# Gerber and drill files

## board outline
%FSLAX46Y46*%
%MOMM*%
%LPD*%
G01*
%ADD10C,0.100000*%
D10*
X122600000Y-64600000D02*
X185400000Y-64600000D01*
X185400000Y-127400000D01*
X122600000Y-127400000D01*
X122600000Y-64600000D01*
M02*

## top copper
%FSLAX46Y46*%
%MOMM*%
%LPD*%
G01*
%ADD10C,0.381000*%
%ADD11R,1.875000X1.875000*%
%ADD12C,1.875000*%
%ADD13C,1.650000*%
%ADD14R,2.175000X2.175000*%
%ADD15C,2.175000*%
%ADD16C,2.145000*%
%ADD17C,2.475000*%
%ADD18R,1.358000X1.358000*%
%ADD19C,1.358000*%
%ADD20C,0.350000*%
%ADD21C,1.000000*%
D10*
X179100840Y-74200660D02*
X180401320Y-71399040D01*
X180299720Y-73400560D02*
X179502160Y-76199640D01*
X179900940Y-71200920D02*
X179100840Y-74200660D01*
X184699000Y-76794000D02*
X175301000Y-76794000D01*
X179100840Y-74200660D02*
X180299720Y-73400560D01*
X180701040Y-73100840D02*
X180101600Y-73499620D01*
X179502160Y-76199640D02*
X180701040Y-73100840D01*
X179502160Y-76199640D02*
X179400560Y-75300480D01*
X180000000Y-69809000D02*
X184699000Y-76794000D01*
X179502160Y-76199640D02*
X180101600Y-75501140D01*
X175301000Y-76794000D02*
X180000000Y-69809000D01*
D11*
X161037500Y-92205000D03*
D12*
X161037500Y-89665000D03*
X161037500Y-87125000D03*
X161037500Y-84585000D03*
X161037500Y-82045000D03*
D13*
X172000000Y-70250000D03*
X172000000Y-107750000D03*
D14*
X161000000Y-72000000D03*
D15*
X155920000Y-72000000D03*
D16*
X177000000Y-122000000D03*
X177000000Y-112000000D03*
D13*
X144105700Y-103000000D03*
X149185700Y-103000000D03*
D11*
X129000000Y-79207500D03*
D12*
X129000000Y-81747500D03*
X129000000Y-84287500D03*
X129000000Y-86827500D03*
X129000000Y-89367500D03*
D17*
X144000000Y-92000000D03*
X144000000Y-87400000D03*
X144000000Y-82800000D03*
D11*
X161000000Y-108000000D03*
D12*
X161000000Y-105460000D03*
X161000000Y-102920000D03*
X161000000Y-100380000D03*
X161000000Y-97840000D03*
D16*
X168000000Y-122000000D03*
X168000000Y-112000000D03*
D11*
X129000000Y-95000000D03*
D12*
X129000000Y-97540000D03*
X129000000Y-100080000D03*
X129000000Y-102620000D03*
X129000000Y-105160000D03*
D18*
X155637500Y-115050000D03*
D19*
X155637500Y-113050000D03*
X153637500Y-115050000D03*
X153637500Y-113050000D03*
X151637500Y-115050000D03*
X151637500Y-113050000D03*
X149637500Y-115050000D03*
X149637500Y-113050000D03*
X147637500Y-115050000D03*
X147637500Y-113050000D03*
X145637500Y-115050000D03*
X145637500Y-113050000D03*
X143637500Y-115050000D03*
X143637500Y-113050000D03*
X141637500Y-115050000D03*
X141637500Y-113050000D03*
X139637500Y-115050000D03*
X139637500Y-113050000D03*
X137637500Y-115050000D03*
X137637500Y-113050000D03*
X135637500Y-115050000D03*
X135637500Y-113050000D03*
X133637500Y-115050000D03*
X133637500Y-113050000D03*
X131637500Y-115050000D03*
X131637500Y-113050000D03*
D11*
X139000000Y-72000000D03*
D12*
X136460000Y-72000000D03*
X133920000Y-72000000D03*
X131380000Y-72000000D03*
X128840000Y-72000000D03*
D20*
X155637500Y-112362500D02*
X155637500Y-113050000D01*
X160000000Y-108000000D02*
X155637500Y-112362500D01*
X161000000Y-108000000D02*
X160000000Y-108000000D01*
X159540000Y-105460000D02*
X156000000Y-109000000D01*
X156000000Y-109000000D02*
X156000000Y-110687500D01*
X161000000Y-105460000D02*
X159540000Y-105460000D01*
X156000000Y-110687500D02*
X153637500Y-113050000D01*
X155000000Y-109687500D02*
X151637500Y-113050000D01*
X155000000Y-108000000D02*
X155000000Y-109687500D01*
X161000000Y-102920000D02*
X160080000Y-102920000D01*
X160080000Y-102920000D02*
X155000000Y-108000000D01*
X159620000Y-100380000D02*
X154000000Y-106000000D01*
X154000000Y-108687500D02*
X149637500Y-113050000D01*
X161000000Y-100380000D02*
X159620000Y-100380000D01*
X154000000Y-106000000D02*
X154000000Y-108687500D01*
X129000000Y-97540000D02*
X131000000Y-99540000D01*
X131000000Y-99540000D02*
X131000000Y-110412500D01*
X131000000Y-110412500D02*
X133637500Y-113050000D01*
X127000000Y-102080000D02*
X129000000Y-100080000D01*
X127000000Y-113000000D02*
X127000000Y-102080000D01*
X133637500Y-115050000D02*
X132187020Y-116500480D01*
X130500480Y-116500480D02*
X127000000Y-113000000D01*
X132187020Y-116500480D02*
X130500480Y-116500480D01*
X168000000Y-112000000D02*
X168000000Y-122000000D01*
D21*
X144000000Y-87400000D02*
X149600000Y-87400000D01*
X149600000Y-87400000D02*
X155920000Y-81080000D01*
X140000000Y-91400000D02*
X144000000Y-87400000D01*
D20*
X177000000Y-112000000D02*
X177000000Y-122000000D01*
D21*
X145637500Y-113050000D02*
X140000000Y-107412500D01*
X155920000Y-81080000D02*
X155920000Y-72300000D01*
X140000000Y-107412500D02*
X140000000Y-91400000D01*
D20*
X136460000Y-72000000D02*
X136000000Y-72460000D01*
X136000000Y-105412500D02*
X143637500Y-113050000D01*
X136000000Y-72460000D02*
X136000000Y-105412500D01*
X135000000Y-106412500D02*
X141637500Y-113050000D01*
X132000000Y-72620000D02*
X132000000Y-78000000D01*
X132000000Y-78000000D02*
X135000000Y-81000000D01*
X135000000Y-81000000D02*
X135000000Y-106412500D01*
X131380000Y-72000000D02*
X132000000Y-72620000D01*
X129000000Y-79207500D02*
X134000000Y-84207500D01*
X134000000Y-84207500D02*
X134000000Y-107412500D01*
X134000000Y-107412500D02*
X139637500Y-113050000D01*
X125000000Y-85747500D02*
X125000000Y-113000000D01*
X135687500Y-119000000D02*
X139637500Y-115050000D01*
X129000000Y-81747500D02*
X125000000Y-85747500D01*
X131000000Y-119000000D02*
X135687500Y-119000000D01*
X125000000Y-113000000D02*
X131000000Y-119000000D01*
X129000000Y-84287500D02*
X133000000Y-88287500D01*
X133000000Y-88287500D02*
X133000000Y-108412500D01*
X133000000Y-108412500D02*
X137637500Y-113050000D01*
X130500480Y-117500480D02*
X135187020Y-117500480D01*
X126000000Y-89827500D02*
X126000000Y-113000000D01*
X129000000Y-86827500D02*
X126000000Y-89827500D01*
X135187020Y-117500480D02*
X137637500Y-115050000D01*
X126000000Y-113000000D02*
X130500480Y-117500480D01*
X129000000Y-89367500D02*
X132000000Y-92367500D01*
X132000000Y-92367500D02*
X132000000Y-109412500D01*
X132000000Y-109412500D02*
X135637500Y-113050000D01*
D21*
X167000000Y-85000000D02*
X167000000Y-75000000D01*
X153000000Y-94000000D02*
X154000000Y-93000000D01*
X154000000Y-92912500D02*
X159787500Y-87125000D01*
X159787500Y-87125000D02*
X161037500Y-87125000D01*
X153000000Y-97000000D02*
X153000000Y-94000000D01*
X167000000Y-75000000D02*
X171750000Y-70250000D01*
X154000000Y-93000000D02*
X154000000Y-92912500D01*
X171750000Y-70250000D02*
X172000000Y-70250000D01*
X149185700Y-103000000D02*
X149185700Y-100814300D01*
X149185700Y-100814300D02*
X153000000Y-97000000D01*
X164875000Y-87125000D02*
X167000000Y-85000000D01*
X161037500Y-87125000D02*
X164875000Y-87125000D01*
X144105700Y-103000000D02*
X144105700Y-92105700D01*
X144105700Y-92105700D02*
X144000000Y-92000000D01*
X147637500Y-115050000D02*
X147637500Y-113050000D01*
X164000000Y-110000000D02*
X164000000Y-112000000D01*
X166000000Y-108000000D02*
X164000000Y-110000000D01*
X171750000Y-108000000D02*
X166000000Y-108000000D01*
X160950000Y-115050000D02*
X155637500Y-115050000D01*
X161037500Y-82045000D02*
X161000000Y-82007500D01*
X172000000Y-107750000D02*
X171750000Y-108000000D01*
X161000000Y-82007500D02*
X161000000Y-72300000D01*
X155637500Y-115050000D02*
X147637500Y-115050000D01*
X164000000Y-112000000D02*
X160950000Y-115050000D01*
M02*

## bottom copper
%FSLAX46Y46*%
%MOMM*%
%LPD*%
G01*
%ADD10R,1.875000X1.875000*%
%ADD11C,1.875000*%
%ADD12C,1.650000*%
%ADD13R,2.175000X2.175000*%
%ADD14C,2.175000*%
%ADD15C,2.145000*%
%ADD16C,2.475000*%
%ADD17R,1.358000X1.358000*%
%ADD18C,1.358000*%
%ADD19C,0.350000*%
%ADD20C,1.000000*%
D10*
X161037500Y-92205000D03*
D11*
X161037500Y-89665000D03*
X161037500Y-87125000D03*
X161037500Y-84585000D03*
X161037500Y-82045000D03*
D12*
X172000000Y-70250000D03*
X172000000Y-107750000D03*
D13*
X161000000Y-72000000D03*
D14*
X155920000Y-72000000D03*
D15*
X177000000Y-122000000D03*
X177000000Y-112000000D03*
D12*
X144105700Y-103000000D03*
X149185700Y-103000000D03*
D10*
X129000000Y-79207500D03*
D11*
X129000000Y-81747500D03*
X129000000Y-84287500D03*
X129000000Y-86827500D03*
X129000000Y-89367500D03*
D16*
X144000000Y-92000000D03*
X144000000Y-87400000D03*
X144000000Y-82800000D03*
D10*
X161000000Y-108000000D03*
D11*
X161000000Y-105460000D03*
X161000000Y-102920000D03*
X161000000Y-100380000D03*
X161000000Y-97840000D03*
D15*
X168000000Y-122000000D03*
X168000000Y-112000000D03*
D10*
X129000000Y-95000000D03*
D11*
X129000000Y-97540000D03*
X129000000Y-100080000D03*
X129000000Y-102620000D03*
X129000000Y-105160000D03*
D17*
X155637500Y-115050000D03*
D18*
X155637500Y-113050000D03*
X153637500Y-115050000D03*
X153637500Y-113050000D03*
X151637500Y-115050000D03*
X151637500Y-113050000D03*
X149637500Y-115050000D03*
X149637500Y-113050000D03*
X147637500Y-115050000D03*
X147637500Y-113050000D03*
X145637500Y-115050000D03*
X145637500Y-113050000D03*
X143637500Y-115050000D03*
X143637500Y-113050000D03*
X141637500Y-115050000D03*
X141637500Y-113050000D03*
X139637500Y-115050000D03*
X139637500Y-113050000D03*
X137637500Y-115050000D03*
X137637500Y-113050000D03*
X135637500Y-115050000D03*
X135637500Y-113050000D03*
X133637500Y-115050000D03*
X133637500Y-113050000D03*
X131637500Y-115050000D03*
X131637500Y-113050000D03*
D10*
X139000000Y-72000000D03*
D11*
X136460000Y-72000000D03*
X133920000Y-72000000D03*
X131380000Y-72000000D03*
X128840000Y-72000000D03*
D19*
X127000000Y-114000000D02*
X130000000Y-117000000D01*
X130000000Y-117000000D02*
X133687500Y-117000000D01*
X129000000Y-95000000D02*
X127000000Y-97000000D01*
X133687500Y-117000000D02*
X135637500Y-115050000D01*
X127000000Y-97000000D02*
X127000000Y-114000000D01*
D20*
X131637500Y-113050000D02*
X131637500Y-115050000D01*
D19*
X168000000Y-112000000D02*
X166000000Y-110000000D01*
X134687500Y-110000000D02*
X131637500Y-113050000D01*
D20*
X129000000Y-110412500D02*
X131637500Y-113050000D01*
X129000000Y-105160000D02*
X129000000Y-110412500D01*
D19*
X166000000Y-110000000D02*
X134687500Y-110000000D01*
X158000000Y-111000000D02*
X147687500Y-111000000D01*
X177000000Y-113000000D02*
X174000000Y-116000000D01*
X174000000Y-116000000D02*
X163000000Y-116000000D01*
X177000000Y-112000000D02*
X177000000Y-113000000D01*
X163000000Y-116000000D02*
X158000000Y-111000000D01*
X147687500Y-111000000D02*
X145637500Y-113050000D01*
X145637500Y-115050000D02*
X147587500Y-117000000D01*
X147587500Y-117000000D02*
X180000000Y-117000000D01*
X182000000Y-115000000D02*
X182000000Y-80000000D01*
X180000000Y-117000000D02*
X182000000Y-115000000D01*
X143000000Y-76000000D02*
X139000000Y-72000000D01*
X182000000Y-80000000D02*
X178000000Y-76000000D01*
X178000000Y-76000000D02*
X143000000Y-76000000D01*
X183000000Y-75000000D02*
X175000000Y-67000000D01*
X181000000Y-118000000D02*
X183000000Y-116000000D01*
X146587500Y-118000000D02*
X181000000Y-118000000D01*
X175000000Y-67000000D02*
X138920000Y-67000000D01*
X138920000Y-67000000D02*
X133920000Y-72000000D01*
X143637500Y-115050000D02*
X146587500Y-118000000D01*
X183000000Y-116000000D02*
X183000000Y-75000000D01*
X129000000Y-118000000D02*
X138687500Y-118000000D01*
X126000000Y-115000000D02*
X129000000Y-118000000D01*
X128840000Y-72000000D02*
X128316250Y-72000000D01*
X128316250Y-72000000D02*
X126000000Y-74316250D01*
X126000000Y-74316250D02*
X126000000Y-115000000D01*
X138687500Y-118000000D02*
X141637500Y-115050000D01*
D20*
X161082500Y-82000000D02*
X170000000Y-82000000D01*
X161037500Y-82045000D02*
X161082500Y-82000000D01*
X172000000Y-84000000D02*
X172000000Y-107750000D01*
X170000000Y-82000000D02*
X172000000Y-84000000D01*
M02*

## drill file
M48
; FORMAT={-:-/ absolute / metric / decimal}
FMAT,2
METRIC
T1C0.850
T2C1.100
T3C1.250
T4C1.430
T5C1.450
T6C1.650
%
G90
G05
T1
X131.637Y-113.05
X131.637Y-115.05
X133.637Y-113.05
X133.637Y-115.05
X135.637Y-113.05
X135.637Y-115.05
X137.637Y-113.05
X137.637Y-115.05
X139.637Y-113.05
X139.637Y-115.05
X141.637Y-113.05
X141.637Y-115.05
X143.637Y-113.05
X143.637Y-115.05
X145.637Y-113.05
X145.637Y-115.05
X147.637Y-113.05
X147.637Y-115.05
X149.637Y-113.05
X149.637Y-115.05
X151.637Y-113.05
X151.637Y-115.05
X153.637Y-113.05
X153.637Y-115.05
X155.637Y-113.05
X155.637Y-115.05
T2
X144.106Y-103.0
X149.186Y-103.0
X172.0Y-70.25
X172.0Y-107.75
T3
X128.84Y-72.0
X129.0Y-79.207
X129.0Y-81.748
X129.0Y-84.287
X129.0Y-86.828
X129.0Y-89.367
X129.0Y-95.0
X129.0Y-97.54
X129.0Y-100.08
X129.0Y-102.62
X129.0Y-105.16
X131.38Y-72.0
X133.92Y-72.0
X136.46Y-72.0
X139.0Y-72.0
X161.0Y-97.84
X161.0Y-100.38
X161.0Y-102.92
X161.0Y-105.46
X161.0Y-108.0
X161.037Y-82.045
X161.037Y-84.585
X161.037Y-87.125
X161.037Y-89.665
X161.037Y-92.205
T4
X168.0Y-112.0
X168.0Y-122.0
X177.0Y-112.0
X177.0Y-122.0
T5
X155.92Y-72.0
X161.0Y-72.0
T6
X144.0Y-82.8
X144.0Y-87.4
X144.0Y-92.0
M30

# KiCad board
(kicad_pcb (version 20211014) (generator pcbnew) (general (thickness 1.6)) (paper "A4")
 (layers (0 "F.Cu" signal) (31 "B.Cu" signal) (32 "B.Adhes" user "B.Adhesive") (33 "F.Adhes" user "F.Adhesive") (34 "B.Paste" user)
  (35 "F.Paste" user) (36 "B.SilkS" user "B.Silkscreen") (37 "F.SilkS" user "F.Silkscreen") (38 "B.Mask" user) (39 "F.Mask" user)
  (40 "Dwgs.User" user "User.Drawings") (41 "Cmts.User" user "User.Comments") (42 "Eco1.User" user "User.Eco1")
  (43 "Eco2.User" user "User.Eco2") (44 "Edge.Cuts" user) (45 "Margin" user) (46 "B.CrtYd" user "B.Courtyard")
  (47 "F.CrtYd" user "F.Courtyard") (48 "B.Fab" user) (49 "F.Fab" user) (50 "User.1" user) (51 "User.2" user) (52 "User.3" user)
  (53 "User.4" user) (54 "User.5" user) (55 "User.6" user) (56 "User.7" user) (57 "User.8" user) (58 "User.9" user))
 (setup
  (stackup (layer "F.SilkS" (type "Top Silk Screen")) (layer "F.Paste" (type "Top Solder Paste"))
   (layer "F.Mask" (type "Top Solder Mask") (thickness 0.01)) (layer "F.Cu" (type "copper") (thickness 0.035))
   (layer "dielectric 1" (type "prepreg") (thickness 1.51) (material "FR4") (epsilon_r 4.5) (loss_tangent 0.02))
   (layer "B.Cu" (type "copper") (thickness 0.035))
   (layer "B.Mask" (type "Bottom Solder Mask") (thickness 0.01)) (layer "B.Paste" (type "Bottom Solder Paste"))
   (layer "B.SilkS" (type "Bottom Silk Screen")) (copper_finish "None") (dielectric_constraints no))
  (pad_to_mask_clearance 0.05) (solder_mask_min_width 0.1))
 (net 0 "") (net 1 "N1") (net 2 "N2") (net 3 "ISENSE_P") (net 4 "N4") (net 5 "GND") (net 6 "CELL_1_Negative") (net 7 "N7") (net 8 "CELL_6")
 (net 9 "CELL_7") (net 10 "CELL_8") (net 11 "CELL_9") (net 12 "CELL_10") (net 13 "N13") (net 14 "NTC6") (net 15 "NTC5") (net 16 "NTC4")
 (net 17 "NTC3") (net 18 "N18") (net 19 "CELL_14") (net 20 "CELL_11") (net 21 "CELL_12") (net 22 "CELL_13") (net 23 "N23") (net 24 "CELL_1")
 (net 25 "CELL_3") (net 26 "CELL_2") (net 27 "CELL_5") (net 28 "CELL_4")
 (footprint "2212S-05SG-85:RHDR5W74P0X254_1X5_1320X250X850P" (layer "F.Cu") (at 161.0375 92.205 90)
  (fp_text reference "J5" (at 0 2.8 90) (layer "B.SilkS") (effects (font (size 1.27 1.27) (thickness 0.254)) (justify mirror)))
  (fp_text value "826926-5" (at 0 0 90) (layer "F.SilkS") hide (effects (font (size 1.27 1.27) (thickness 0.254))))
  (pad "1" thru_hole rect locked (at 0 0 90) (size 1.875 1.875) (drill 1.25) (layers *.Cu *.Mask) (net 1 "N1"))
  (pad "2" thru_hole circle locked (at 2.54 0 90) (size 1.875 1.875) (drill 1.25) (layers *.Cu *.Mask) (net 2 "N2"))
  (pad "3" thru_hole circle locked (at 5.08 0 90) (size 1.875 1.875) (drill 1.25) (layers *.Cu *.Mask) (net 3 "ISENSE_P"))
  (pad "4" thru_hole circle locked (at 7.62 0 90) (size 1.875 1.875) (drill 1.25) (layers *.Cu *.Mask) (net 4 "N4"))
  (pad "5" thru_hole circle locked (at 10.16 0 90) (size 1.875 1.875) (drill 1.25) (layers *.Cu *.Mask) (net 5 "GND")))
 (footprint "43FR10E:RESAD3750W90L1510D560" (layer "F.Cu") (at 172 70.25 -90)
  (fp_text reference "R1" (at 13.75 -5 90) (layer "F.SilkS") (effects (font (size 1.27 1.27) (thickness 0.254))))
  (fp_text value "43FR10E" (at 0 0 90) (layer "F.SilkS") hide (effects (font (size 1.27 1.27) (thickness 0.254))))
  (pad "1" thru_hole circle locked (at 0 0 270) (size 1.65 1.65) (drill 1.1) (layers *.Cu *.Mask) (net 3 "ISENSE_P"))
  (pad "2" thru_hole circle locked (at 37.5 0 270) (size 1.65 1.65) (drill 1.1) (layers *.Cu *.Mask) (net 5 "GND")))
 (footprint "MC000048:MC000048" (layer "F.Cu") (at 161 72 180)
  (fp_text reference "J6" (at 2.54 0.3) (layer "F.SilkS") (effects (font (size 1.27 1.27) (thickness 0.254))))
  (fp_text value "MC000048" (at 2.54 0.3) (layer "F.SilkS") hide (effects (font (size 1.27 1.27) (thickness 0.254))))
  (pad "1" thru_hole rect locked (at 0 0 180) (size 2.175 2.175) (drill 1.45) (layers *.Cu *.Mask) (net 5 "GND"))
  (pad "2" thru_hole circle locked (at 5.08 0 180) (size 2.175 2.175) (drill 1.45) (layers *.Cu *.Mask) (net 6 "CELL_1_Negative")))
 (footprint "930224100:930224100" (layer "F.Cu") (at 177 122 90)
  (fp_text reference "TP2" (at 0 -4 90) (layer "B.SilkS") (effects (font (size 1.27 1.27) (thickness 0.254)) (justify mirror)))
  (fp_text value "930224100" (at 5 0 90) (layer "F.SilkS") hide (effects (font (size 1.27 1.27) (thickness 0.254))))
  (pad "1" thru_hole circle locked (at 0 0 90) (size 2.145 2.145) (drill 1.43) (layers *.Cu *.Mask) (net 6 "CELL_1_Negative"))
  (pad "2" thru_hole circle locked (at 10 0 90) (size 2.145 2.145) (drill 1.43) (layers *.Cu *.Mask) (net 6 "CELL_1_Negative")))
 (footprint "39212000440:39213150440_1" (layer "F.Cu") (at 146.6457 103)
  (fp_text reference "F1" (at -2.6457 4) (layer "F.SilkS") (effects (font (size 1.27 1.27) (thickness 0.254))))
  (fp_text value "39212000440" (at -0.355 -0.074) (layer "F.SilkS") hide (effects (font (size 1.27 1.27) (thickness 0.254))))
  (pad "1" thru_hole circle locked (at -2.54 0) (size 1.65 1.65) (drill 1.1) (layers *.Cu *.Mask) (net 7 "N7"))
  (pad "2" thru_hole circle locked (at 2.54 0) (size 1.65 1.65) (drill 1.1) (layers *.Cu *.Mask) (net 3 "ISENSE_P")))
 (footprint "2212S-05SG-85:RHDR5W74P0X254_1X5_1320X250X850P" (layer "F.Cu") (at 129 79.2075 -90)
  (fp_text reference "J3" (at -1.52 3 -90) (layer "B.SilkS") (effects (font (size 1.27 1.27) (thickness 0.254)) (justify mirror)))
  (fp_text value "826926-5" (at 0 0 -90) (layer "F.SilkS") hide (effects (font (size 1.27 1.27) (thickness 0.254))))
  (pad "1" thru_hole rect locked (at 0 0 270) (size 1.875 1.875) (drill 1.25) (layers *.Cu *.Mask) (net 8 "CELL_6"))
  (pad "2" thru_hole circle locked (at 2.54 0 270) (size 1.875 1.875) (drill 1.25) (layers *.Cu *.Mask) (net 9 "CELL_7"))
  (pad "3" thru_hole circle locked (at 5.08 0 270) (size 1.875 1.875) (drill 1.25) (layers *.Cu *.Mask) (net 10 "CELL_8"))
  (pad "4" thru_hole circle locked (at 7.62 0 270) (size 1.875 1.875) (drill 1.25) (layers *.Cu *.Mask) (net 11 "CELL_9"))
  (pad "5" thru_hole circle locked (at 10.16 0 270) (size 1.875 1.875) (drill 1.25) (layers *.Cu *.Mask) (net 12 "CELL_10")))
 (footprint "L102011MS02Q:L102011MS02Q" (layer "F.Cu") (at 144 92)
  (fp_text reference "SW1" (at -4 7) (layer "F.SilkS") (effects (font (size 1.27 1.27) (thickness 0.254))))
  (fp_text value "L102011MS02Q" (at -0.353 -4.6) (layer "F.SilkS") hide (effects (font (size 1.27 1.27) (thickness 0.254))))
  (pad "1" thru_hole circle locked (at 0 0) (size 2.475 2.475) (drill 1.65) (layers *.Cu *.Mask) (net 7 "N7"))
  (pad "2" thru_hole circle locked (at 0 -4.6) (size 2.475 2.475) (drill 1.65) (layers *.Cu *.Mask) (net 6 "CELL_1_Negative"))
  (pad "3" thru_hole circle locked (at 0 -9.2) (size 2.475 2.475) (drill 1.65) (layers *.Cu *.Mask) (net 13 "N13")))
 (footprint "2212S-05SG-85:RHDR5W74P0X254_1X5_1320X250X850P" (layer "F.Cu") (at 161 108 90)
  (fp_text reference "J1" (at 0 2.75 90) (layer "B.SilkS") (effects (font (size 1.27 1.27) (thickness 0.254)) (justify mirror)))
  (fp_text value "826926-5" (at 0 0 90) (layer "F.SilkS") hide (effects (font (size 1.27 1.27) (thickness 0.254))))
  (pad "1" thru_hole rect locked (at 0 0 90) (size 1.875 1.875) (drill 1.25) (layers *.Cu *.Mask) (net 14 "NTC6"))
  (pad "2" thru_hole circle locked (at 2.54 0 90) (size 1.875 1.875) (drill 1.25) (layers *.Cu *.Mask) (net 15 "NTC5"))
  (pad "3" thru_hole circle locked (at 5.08 0 90) (size 1.875 1.875) (drill 1.25) (layers *.Cu *.Mask) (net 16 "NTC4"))
  (pad "4" thru_hole circle locked (at 7.62 0 90) (size 1.875 1.875) (drill 1.25) (layers *.Cu *.Mask) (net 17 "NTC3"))
  (pad "5" thru_hole circle locked (at 10.16 0 90) (size 1.875 1.875) (drill 1.25) (layers *.Cu *.Mask) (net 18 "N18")))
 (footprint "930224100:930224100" (layer "F.Cu") (at 168 122 90)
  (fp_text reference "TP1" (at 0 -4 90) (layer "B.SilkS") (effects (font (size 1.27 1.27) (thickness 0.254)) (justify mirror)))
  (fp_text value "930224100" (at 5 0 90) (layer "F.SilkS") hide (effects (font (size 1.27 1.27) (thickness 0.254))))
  (pad "1" thru_hole circle locked (at 0 0 90) (size 2.145 2.145) (drill 1.43) (layers *.Cu *.Mask) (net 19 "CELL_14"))
  (pad "2" thru_hole circle locked (at 10 0 90) (size 2.145 2.145) (drill 1.43) (layers *.Cu *.Mask) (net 19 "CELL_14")))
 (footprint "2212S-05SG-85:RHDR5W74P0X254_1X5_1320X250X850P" (layer "F.Cu") (at 129 95 -90)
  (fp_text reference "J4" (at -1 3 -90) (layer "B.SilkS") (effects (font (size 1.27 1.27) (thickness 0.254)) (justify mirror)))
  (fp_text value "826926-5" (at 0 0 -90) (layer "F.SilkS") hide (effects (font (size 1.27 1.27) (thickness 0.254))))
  (pad "1" thru_hole rect locked (at 0 0 270) (size 1.875 1.875) (drill 1.25) (layers *.Cu *.Mask) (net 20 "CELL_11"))
  (pad "2" thru_hole circle locked (at 2.54 0 270) (size 1.875 1.875) (drill 1.25) (layers *.Cu *.Mask) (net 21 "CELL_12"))
  (pad "3" thru_hole circle locked (at 5.08 0 270) (size 1.875 1.875) (drill 1.25) (layers *.Cu *.Mask) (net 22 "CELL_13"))
  (pad "4" thru_hole circle locked (at 7.62 0 270) (size 1.875 1.875) (drill 1.25) (layers *.Cu *.Mask) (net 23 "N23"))
  (pad "5" thru_hole circle locked (at 10.16 0 270) (size 1.875 1.875) (drill 1.25) (layers *.Cu *.Mask) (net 19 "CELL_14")))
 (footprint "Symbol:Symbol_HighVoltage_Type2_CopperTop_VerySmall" (layer "F.Cu") (at 180 74)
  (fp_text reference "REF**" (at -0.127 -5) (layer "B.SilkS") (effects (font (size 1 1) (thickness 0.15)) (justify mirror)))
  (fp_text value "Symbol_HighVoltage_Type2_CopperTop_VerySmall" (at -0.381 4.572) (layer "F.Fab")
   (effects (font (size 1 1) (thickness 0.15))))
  (fp_line (start -0.89916 0.20066) (end 0.40132 -2.60096) (layer "F.Cu") (width 0.381))
  (fp_line (start 0.29972 -0.59944) (end -0.49784 2.19964) (layer "F.Cu") (width 0.381))
  (fp_line (start -0.09906 -2.79908) (end -0.89916 0.20066) (layer "F.Cu") (width 0.381))
  (fp_line (start 4.699 2.794) (end -4.699 2.794) (layer "F.Cu") (width 0.381))
  (fp_line (start -0.89916 0.20066) (end 0.29972 -0.59944) (layer "F.Cu") (width 0.381))
  (fp_line (start 0.70104 -0.89916) (end 0.1016 -0.50038) (layer "F.Cu") (width 0.381))
  (fp_line (start -0.49784 2.19964) (end 0.70104 -0.89916) (layer "F.Cu") (width 0.381))
  (fp_line (start -0.49784 2.19964) (end -0.59944 1.30048) (layer "F.Cu") (width 0.381))
  (fp_line (start 0 -4.191) (end 4.699 2.794) (layer "F.Cu") (width 0.381))
  (fp_line (start -0.49784 2.19964) (end 0.1016 1.50114) (layer "F.Cu") (width 0.381))
  (fp_line (start -4.699 2.794) (end 0 -4.191) (layer "F.Cu") (width 0.381)))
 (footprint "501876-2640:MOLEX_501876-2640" (layer "F.Cu") (at 143.6375 115.05)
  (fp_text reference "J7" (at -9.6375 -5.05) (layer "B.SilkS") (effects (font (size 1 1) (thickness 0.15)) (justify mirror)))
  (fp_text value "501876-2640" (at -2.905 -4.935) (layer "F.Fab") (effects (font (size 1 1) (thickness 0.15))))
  (pad "1" thru_hole rect locked (at 12 0) (size 1.358 1.358) (drill 0.85) (layers *.Cu *.Mask) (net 5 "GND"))
  (pad "2" thru_hole circle locked (at 12 -2) (size 1.358 1.358) (drill 0.85) (layers *.Cu *.Mask) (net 14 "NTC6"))
  (pad "3" thru_hole circle locked (at 10 0) (size 1.358 1.358) (drill 0.85) (layers *.Cu *.Mask) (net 5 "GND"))
  (pad "4" thru_hole circle locked (at 10 -2) (size 1.358 1.358) (drill 0.85) (layers *.Cu *.Mask) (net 15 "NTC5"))
  (pad "5" thru_hole circle locked (at 8 0) (size 1.358 1.358) (drill 0.85) (layers *.Cu *.Mask) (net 5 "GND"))
  (pad "6" thru_hole circle locked (at 8 -2) (size 1.358 1.358) (drill 0.85) (layers *.Cu *.Mask) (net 16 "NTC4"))
  (pad "7" thru_hole circle locked (at 6 0) (size 1.358 1.358) (drill 0.85) (layers *.Cu *.Mask) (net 5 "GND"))
  (pad "8" thru_hole circle locked (at 6 -2) (size 1.358 1.358) (drill 0.85) (layers *.Cu *.Mask) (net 17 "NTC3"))
  (pad "9" thru_hole circle locked (at 4 0) (size 1.358 1.358) (drill 0.85) (layers *.Cu *.Mask) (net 5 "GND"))
  (pad "10" thru_hole circle locked (at 4 -2) (size 1.358 1.358) (drill 0.85) (layers *.Cu *.Mask) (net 5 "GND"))
  (pad "11" thru_hole circle locked (at 2 0) (size 1.358 1.358) (drill 0.85) (layers *.Cu *.Mask) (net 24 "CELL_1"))
  (pad "12" thru_hole circle locked (at 2 -2) (size 1.358 1.358) (drill 0.85) (layers *.Cu *.Mask) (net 6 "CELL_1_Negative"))
  (pad "13" thru_hole circle locked (at 0 0) (size 1.358 1.358) (drill 0.85) (layers *.Cu *.Mask) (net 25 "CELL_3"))
  (pad "14" thru_hole circle locked (at 0 -2) (size 1.358 1.358) (drill 0.85) (layers *.Cu *.Mask) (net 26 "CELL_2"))
  (pad "15" thru_hole circle locked (at -2 0) (size 1.358 1.358) (drill 0.85) (layers *.Cu *.Mask) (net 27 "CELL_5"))
  (pad "16" thru_hole circle locked (at -2 -2) (size 1.358 1.358) (drill 0.85) (layers *.Cu *.Mask) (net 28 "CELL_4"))
  (pad "17" thru_hole circle locked (at -4 0) (size 1.358 1.358) (drill 0.85) (layers *.Cu *.Mask) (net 9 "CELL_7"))
  (pad "18" thru_hole circle locked (at -4 -2) (size 1.358 1.358) (drill 0.85) (layers *.Cu *.Mask) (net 8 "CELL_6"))
  (pad "19" thru_hole circle locked (at -6 0) (size 1.358 1.358) (drill 0.85) (layers *.Cu *.Mask) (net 11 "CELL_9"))
  (pad "20" thru_hole circle locked (at -6 -2) (size 1.358 1.358) (drill 0.85) (layers *.Cu *.Mask) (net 10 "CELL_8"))
  (pad "21" thru_hole circle locked (at -8 0) (size 1.358 1.358) (drill 0.85) (layers *.Cu *.Mask) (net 20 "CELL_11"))
  (pad "22" thru_hole circle locked (at -8 -2) (size 1.358 1.358) (drill 0.85) (layers *.Cu *.Mask) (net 12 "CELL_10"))
  (pad "23" thru_hole circle locked (at -10 0) (size 1.358 1.358) (drill 0.85) (layers *.Cu *.Mask) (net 22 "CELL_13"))
  (pad "24" thru_hole circle locked (at -10 -2) (size 1.358 1.358) (drill 0.85) (layers *.Cu *.Mask) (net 21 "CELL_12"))
  (pad "25" thru_hole circle locked (at -12 0) (size 1.358 1.358) (drill 0.85) (layers *.Cu *.Mask) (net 19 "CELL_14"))
  (pad "26" thru_hole circle locked (at -12 -2) (size 1.358 1.358) (drill 0.85) (layers *.Cu *.Mask) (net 19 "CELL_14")))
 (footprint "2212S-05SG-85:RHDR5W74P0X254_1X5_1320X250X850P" (layer "F.Cu") (at 139 72 180)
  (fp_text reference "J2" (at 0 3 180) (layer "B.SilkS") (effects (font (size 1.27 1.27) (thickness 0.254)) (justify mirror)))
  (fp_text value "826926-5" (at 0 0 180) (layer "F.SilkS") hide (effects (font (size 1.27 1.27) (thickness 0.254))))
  (pad "1" thru_hole rect locked (at 0 0 180) (size 1.875 1.875) (drill 1.25) (layers *.Cu *.Mask) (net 24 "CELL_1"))
  (pad "2" thru_hole circle locked (at 2.54 0 180) (size 1.875 1.875) (drill 1.25) (layers *.Cu *.Mask) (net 26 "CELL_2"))
  (pad "3" thru_hole circle locked (at 5.08 0 180) (size 1.875 1.875) (drill 1.25) (layers *.Cu *.Mask) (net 25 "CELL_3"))
  (pad "4" thru_hole circle locked (at 7.62 0 180) (size 1.875 1.875) (drill 1.25) (layers *.Cu *.Mask) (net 28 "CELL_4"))
  (pad "5" thru_hole circle locked (at 10.16 0 180) (size 1.875 1.875) (drill 1.25) (layers *.Cu *.Mask) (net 27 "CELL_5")))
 (gr_rect (start 122.6 64.6) (end 185.4 127.4) (layer "Edge.Cuts") (width 0.1) (fill none))
 (segment (start 155.6375 112.3625) (end 155.6375 113.05) (width 0.35) (layer "F.Cu") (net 14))
 (segment (start 160 108) (end 155.6375 112.3625) (width 0.35) (layer "F.Cu") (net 14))
 (segment (start 161 108) (end 160 108) (width 0.35) (layer "F.Cu") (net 14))
 (segment (start 159.54 105.46) (end 156 109) (width 0.35) (layer "F.Cu") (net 15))
 (segment (start 156 109) (end 156 110.6875) (width 0.35) (layer "F.Cu") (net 15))
 (segment (start 161 105.46) (end 159.54 105.46) (width 0.35) (layer "F.Cu") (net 15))
 (segment (start 156 110.6875) (end 153.6375 113.05) (width 0.35) (layer "F.Cu") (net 15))
 (segment (start 155 109.6875) (end 151.6375 113.05) (width 0.35) (layer "F.Cu") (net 16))
 (segment (start 155 108) (end 155 109.6875) (width 0.35) (layer "F.Cu") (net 16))
 (segment (start 161 102.92) (end 160.08 102.92) (width 0.35) (layer "F.Cu") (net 16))
 (segment (start 160.08 102.92) (end 155 108) (width 0.35) (layer "F.Cu") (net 16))
 (segment (start 159.62 100.38) (end 154 106) (width 0.35) (layer "F.Cu") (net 17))
 (segment (start 154 108.6875) (end 149.6375 113.05) (width 0.35) (layer "F.Cu") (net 17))
 (segment (start 161 100.38) (end 159.62 100.38) (width 0.35) (layer "F.Cu") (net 17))
 (segment (start 154 106) (end 154 108.6875) (width 0.35) (layer "F.Cu") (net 17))
 (segment (start 127 114) (end 130 117) (width 0.35) (layer "B.Cu") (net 20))
 (segment (start 130 117) (end 133.6875 117) (width 0.35) (layer "B.Cu") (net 20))
 (segment (start 129 95) (end 127 97) (width 0.35) (layer "B.Cu") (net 20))
 (segment (start 133.6875 117) (end 135.6375 115.05) (width 0.35) (layer "B.Cu") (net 20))
 (segment (start 127 97) (end 127 114) (width 0.35) (layer "B.Cu") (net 20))
 (segment (start 129 97.54) (end 131 99.54) (width 0.35) (layer "F.Cu") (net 21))
 (segment (start 131 99.54) (end 131 110.4125) (width 0.35) (layer "F.Cu") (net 21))
 (segment (start 131 110.4125) (end 133.6375 113.05) (width 0.35) (layer "F.Cu") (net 21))
 (segment (start 127 102.08) (end 129 100.08) (width 0.35) (layer "F.Cu") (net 22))
 (segment (start 127 113) (end 127 102.08) (width 0.35) (layer "F.Cu") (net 22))
 (segment (start 133.6375 115.05) (end 132.18702 116.50048) (width 0.35) (layer "F.Cu") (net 22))
 (segment (start 130.50048 116.50048) (end 127 113) (width 0.35) (layer "F.Cu") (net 22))
 (segment (start 132.18702 116.50048) (end 130.50048 116.50048) (width 0.35) (layer "F.Cu") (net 22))
 (segment (start 168 112) (end 168 122) (width 0.35) (layer "F.Cu") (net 19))
 (segment (start 131.6375 113.05) (end 131.6375 115.05) (width 1) (layer "B.Cu") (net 19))
 (segment (start 168 112) (end 166 110) (width 0.35) (layer "B.Cu") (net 19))
 (segment (start 134.6875 110) (end 131.6375 113.05) (width 0.35) (layer "B.Cu") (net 19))
 (segment (start 129 110.4125) (end 131.6375 113.05) (width 1) (layer "B.Cu") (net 19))
 (segment (start 129 105.16) (end 129 110.4125) (width 1) (layer "B.Cu") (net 19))
 (segment (start 166 110) (end 134.6875 110) (width 0.35) (layer "B.Cu") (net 19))
 (segment (start 144 87.4) (end 149.6 87.4) (width 1) (layer "F.Cu") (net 6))
 (segment (start 149.6 87.4) (end 155.92 81.08) (width 1) (layer "F.Cu") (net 6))
 (segment (start 140 91.4) (end 144 87.4) (width 1) (layer "F.Cu") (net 6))
 (segment (start 177 112) (end 177 122) (width 0.35) (layer "F.Cu") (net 6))
 (segment (start 145.6375 113.05) (end 140 107.4125) (width 1) (layer "F.Cu") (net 6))
 (segment (start 155.92 81.08) (end 155.92 72.3) (width 1) (layer "F.Cu") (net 6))
 (segment (start 140 107.4125) (end 140 91.4) (width 1) (layer "F.Cu") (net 6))
 (segment (start 158 111) (end 147.6875 111) (width 0.35) (layer "B.Cu") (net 6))
 (segment (start 177 113) (end 174 116) (width 0.35) (layer "B.Cu") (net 6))
 (segment (start 174 116) (end 163 116) (width 0.35) (layer "B.Cu") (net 6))
 (segment (start 177 112) (end 177 113) (width 0.35) (layer "B.Cu") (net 6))
 (segment (start 163 116) (end 158 111) (width 0.35) (layer "B.Cu") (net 6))
 (segment (start 147.6875 111) (end 145.6375 113.05) (width 0.35) (layer "B.Cu") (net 6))
 (segment (start 145.6375 115.05) (end 147.5875 117) (width 0.35) (layer "B.Cu") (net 24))
 (segment (start 147.5875 117) (end 180 117) (width 0.35) (layer "B.Cu") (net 24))
 (segment (start 182 115) (end 182 80) (width 0.35) (layer "B.Cu") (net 24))
 (segment (start 180 117) (end 182 115) (width 0.35) (layer "B.Cu") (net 24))
 (segment (start 143 76) (end 139 72) (width 0.35) (layer "B.Cu") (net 24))
 (segment (start 182 80) (end 178 76) (width 0.35) (layer "B.Cu") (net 24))
 (segment (start 178 76) (end 143 76) (width 0.35) (layer "B.Cu") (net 24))
 (segment (start 136.46 72) (end 136 72.46) (width 0.35) (layer "F.Cu") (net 26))
 (segment (start 136 105.4125) (end 143.6375 113.05) (width 0.35) (layer "F.Cu") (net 26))
 (segment (start 136 72.46) (end 136 105.4125) (width 0.35) (layer "F.Cu") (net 26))
 (segment (start 183 75) (end 175 67) (width 0.35) (layer "B.Cu") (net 25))
 (segment (start 181 118) (end 183 116) (width 0.35) (layer "B.Cu") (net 25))
 (segment (start 146.5875 118) (end 181 118) (width 0.35) (layer "B.Cu") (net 25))
 (segment (start 175 67) (end 138.92 67) (width 0.35) (layer "B.Cu") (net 25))
 (segment (start 138.92 67) (end 133.92 72) (width 0.35) (layer "B.Cu") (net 25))
 (segment (start 143.6375 115.05) (end 146.5875 118) (width 0.35) (layer "B.Cu") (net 25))
 (segment (start 183 116) (end 183 75) (width 0.35) (layer "B.Cu") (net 25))
 (segment (start 135 106.4125) (end 141.6375 113.05) (width 0.35) (layer "F.Cu") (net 28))
 (segment (start 132 72.62) (end 132 78) (width 0.35) (layer "F.Cu") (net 28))
 (segment (start 132 78) (end 135 81) (width 0.35) (layer "F.Cu") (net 28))
 (segment (start 135 81) (end 135 106.4125) (width 0.35) (layer "F.Cu") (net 28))
 (segment (start 131.38 72) (end 132 72.62) (width 0.35) (layer "F.Cu") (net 28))
 (segment (start 129 118) (end 138.6875 118) (width 0.35) (layer "B.Cu") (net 27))
 (segment (start 126 115) (end 129 118) (width 0.35) (layer "B.Cu") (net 27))
 (segment (start 128.84 72) (end 128.31625 72) (width 0.35) (layer "B.Cu") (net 27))
 (segment (start 128.31625 72) (end 126 74.31625) (width 0.35) (layer "B.Cu") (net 27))
 (segment (start 126 74.31625) (end 126 115) (width 0.35) (layer "B.Cu") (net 27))
 (segment (start 138.6875 118) (end 141.6375 115.05) (width 0.35) (layer "B.Cu") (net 27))
 (segment (start 129 79.2075) (end 134 84.2075) (width 0.35) (layer "F.Cu") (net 8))
 (segment (start 134 84.2075) (end 134 107.4125) (width 0.35) (layer "F.Cu") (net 8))
 (segment (start 134 107.4125) (end 139.6375 113.05) (width 0.35) (layer "F.Cu") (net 8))
 (segment (start 125 85.7475) (end 125 113) (width 0.35) (layer "F.Cu") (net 9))
 (segment (start 135.6875 119) (end 139.6375 115.05) (width 0.35) (layer "F.Cu") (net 9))
 (segment (start 129 81.7475) (end 125 85.7475) (width 0.35) (layer "F.Cu") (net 9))
 (segment (start 131 119) (end 135.6875 119) (width 0.35) (layer "F.Cu") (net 9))
 (segment (start 125 113) (end 131 119) (width 0.35) (layer "F.Cu") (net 9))
 (segment (start 129 84.2875) (end 133 88.2875) (width 0.35) (layer "F.Cu") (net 10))
 (segment (start 133 88.2875) (end 133 108.4125) (width 0.35) (layer "F.Cu") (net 10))
 (segment (start 133 108.4125) (end 137.6375 113.05) (width 0.35) (layer "F.Cu") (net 10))
 (segment (start 130.50048 117.50048) (end 135.18702 117.50048) (width 0.35) (layer "F.Cu") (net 11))
 (segment (start 126 89.8275) (end 126 113) (width 0.35) (layer "F.Cu") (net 11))
 (segment (start 129 86.8275) (end 126 89.8275) (width 0.35) (layer "F.Cu") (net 11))
 (segment (start 135.18702 117.50048) (end 137.6375 115.05) (width 0.35) (layer "F.Cu") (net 11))
 (segment (start 126 113) (end 130.50048 117.50048) (width 0.35) (layer "F.Cu") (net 11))
 (segment (start 129 89.3675) (end 132 92.3675) (width 0.35) (layer "F.Cu") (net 12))
 (segment (start 132 92.3675) (end 132 109.4125) (width 0.35) (layer "F.Cu") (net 12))
 (segment (start 132 109.4125) (end 135.6375 113.05) (width 0.35) (layer "F.Cu") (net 12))
 (segment (start 167 85) (end 167 75) (width 1) (layer "F.Cu") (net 3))
 (segment (start 153 94) (end 154 93) (width 1) (layer "F.Cu") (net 3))
 (segment (start 154 92.9125) (end 159.7875 87.125) (width 1) (layer "F.Cu") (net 3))
 (segment (start 159.7875 87.125) (end 161.0375 87.125) (width 1) (layer "F.Cu") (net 3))
 (segment (start 153 97) (end 153 94) (width 1) (layer "F.Cu") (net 3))
 (segment (start 167 75) (end 171.75 70.25) (width 1) (layer "F.Cu") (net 3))
 (segment (start 154 93) (end 154 92.9125) (width 1) (layer "F.Cu") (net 3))
 (segment (start 171.75 70.25) (end 172 70.25) (width 1) (layer "F.Cu") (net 3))
 (segment (start 149.1857 103) (end 149.1857 100.8143) (width 1) (layer "F.Cu") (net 3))
 (segment (start 149.1857 100.8143) (end 153 97) (width 1) (layer "F.Cu") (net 3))
 (segment (start 164.875 87.125) (end 167 85) (width 1) (layer "F.Cu") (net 3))
 (segment (start 161.0375 87.125) (end 164.875 87.125) (width 1) (layer "F.Cu") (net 3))
 (segment (start 144.1057 103) (end 144.1057 92.1057) (width 1) (layer "F.Cu") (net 7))
 (segment (start 144.1057 92.1057) (end 144 92) (width 1) (layer "F.Cu") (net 7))
 (segment (start 147.6375 115.05) (end 147.6375 113.05) (width 1) (layer "F.Cu") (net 5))
 (segment (start 164 110) (end 164 112) (width 1) (layer "F.Cu") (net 5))
 (segment (start 166 108) (end 164 110) (width 1) (layer "F.Cu") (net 5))
 (segment (start 171.75 108) (end 166 108) (width 1) (layer "F.Cu") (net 5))
 (segment (start 160.95 115.05) (end 155.6375 115.05) (width 1) (layer "F.Cu") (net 5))
 (segment (start 161.0375 82.045) (end 161 82.0075) (width 1) (layer "F.Cu") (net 5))
 (segment (start 172 107.75) (end 171.75 108) (width 1) (layer "F.Cu") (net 5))
 (segment (start 161 82.0075) (end 161 72.3) (width 1) (layer "F.Cu") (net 5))
 (segment (start 155.6375 115.05) (end 147.6375 115.05) (width 1) (layer "F.Cu") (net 5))
 (segment (start 164 112) (end 160.95 115.05) (width 1) (layer "F.Cu") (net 5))
 (segment (start 161.0825 82) (end 170 82) (width 1) (layer "B.Cu") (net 5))
 (segment (start 161.0375 82.045) (end 161.0825 82) (width 1) (layer "B.Cu") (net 5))
 (segment (start 172 84) (end 172 107.75) (width 1) (layer "B.Cu") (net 5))
 (segment (start 170 82) (end 172 84) (width 1) (layer "B.Cu") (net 5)))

